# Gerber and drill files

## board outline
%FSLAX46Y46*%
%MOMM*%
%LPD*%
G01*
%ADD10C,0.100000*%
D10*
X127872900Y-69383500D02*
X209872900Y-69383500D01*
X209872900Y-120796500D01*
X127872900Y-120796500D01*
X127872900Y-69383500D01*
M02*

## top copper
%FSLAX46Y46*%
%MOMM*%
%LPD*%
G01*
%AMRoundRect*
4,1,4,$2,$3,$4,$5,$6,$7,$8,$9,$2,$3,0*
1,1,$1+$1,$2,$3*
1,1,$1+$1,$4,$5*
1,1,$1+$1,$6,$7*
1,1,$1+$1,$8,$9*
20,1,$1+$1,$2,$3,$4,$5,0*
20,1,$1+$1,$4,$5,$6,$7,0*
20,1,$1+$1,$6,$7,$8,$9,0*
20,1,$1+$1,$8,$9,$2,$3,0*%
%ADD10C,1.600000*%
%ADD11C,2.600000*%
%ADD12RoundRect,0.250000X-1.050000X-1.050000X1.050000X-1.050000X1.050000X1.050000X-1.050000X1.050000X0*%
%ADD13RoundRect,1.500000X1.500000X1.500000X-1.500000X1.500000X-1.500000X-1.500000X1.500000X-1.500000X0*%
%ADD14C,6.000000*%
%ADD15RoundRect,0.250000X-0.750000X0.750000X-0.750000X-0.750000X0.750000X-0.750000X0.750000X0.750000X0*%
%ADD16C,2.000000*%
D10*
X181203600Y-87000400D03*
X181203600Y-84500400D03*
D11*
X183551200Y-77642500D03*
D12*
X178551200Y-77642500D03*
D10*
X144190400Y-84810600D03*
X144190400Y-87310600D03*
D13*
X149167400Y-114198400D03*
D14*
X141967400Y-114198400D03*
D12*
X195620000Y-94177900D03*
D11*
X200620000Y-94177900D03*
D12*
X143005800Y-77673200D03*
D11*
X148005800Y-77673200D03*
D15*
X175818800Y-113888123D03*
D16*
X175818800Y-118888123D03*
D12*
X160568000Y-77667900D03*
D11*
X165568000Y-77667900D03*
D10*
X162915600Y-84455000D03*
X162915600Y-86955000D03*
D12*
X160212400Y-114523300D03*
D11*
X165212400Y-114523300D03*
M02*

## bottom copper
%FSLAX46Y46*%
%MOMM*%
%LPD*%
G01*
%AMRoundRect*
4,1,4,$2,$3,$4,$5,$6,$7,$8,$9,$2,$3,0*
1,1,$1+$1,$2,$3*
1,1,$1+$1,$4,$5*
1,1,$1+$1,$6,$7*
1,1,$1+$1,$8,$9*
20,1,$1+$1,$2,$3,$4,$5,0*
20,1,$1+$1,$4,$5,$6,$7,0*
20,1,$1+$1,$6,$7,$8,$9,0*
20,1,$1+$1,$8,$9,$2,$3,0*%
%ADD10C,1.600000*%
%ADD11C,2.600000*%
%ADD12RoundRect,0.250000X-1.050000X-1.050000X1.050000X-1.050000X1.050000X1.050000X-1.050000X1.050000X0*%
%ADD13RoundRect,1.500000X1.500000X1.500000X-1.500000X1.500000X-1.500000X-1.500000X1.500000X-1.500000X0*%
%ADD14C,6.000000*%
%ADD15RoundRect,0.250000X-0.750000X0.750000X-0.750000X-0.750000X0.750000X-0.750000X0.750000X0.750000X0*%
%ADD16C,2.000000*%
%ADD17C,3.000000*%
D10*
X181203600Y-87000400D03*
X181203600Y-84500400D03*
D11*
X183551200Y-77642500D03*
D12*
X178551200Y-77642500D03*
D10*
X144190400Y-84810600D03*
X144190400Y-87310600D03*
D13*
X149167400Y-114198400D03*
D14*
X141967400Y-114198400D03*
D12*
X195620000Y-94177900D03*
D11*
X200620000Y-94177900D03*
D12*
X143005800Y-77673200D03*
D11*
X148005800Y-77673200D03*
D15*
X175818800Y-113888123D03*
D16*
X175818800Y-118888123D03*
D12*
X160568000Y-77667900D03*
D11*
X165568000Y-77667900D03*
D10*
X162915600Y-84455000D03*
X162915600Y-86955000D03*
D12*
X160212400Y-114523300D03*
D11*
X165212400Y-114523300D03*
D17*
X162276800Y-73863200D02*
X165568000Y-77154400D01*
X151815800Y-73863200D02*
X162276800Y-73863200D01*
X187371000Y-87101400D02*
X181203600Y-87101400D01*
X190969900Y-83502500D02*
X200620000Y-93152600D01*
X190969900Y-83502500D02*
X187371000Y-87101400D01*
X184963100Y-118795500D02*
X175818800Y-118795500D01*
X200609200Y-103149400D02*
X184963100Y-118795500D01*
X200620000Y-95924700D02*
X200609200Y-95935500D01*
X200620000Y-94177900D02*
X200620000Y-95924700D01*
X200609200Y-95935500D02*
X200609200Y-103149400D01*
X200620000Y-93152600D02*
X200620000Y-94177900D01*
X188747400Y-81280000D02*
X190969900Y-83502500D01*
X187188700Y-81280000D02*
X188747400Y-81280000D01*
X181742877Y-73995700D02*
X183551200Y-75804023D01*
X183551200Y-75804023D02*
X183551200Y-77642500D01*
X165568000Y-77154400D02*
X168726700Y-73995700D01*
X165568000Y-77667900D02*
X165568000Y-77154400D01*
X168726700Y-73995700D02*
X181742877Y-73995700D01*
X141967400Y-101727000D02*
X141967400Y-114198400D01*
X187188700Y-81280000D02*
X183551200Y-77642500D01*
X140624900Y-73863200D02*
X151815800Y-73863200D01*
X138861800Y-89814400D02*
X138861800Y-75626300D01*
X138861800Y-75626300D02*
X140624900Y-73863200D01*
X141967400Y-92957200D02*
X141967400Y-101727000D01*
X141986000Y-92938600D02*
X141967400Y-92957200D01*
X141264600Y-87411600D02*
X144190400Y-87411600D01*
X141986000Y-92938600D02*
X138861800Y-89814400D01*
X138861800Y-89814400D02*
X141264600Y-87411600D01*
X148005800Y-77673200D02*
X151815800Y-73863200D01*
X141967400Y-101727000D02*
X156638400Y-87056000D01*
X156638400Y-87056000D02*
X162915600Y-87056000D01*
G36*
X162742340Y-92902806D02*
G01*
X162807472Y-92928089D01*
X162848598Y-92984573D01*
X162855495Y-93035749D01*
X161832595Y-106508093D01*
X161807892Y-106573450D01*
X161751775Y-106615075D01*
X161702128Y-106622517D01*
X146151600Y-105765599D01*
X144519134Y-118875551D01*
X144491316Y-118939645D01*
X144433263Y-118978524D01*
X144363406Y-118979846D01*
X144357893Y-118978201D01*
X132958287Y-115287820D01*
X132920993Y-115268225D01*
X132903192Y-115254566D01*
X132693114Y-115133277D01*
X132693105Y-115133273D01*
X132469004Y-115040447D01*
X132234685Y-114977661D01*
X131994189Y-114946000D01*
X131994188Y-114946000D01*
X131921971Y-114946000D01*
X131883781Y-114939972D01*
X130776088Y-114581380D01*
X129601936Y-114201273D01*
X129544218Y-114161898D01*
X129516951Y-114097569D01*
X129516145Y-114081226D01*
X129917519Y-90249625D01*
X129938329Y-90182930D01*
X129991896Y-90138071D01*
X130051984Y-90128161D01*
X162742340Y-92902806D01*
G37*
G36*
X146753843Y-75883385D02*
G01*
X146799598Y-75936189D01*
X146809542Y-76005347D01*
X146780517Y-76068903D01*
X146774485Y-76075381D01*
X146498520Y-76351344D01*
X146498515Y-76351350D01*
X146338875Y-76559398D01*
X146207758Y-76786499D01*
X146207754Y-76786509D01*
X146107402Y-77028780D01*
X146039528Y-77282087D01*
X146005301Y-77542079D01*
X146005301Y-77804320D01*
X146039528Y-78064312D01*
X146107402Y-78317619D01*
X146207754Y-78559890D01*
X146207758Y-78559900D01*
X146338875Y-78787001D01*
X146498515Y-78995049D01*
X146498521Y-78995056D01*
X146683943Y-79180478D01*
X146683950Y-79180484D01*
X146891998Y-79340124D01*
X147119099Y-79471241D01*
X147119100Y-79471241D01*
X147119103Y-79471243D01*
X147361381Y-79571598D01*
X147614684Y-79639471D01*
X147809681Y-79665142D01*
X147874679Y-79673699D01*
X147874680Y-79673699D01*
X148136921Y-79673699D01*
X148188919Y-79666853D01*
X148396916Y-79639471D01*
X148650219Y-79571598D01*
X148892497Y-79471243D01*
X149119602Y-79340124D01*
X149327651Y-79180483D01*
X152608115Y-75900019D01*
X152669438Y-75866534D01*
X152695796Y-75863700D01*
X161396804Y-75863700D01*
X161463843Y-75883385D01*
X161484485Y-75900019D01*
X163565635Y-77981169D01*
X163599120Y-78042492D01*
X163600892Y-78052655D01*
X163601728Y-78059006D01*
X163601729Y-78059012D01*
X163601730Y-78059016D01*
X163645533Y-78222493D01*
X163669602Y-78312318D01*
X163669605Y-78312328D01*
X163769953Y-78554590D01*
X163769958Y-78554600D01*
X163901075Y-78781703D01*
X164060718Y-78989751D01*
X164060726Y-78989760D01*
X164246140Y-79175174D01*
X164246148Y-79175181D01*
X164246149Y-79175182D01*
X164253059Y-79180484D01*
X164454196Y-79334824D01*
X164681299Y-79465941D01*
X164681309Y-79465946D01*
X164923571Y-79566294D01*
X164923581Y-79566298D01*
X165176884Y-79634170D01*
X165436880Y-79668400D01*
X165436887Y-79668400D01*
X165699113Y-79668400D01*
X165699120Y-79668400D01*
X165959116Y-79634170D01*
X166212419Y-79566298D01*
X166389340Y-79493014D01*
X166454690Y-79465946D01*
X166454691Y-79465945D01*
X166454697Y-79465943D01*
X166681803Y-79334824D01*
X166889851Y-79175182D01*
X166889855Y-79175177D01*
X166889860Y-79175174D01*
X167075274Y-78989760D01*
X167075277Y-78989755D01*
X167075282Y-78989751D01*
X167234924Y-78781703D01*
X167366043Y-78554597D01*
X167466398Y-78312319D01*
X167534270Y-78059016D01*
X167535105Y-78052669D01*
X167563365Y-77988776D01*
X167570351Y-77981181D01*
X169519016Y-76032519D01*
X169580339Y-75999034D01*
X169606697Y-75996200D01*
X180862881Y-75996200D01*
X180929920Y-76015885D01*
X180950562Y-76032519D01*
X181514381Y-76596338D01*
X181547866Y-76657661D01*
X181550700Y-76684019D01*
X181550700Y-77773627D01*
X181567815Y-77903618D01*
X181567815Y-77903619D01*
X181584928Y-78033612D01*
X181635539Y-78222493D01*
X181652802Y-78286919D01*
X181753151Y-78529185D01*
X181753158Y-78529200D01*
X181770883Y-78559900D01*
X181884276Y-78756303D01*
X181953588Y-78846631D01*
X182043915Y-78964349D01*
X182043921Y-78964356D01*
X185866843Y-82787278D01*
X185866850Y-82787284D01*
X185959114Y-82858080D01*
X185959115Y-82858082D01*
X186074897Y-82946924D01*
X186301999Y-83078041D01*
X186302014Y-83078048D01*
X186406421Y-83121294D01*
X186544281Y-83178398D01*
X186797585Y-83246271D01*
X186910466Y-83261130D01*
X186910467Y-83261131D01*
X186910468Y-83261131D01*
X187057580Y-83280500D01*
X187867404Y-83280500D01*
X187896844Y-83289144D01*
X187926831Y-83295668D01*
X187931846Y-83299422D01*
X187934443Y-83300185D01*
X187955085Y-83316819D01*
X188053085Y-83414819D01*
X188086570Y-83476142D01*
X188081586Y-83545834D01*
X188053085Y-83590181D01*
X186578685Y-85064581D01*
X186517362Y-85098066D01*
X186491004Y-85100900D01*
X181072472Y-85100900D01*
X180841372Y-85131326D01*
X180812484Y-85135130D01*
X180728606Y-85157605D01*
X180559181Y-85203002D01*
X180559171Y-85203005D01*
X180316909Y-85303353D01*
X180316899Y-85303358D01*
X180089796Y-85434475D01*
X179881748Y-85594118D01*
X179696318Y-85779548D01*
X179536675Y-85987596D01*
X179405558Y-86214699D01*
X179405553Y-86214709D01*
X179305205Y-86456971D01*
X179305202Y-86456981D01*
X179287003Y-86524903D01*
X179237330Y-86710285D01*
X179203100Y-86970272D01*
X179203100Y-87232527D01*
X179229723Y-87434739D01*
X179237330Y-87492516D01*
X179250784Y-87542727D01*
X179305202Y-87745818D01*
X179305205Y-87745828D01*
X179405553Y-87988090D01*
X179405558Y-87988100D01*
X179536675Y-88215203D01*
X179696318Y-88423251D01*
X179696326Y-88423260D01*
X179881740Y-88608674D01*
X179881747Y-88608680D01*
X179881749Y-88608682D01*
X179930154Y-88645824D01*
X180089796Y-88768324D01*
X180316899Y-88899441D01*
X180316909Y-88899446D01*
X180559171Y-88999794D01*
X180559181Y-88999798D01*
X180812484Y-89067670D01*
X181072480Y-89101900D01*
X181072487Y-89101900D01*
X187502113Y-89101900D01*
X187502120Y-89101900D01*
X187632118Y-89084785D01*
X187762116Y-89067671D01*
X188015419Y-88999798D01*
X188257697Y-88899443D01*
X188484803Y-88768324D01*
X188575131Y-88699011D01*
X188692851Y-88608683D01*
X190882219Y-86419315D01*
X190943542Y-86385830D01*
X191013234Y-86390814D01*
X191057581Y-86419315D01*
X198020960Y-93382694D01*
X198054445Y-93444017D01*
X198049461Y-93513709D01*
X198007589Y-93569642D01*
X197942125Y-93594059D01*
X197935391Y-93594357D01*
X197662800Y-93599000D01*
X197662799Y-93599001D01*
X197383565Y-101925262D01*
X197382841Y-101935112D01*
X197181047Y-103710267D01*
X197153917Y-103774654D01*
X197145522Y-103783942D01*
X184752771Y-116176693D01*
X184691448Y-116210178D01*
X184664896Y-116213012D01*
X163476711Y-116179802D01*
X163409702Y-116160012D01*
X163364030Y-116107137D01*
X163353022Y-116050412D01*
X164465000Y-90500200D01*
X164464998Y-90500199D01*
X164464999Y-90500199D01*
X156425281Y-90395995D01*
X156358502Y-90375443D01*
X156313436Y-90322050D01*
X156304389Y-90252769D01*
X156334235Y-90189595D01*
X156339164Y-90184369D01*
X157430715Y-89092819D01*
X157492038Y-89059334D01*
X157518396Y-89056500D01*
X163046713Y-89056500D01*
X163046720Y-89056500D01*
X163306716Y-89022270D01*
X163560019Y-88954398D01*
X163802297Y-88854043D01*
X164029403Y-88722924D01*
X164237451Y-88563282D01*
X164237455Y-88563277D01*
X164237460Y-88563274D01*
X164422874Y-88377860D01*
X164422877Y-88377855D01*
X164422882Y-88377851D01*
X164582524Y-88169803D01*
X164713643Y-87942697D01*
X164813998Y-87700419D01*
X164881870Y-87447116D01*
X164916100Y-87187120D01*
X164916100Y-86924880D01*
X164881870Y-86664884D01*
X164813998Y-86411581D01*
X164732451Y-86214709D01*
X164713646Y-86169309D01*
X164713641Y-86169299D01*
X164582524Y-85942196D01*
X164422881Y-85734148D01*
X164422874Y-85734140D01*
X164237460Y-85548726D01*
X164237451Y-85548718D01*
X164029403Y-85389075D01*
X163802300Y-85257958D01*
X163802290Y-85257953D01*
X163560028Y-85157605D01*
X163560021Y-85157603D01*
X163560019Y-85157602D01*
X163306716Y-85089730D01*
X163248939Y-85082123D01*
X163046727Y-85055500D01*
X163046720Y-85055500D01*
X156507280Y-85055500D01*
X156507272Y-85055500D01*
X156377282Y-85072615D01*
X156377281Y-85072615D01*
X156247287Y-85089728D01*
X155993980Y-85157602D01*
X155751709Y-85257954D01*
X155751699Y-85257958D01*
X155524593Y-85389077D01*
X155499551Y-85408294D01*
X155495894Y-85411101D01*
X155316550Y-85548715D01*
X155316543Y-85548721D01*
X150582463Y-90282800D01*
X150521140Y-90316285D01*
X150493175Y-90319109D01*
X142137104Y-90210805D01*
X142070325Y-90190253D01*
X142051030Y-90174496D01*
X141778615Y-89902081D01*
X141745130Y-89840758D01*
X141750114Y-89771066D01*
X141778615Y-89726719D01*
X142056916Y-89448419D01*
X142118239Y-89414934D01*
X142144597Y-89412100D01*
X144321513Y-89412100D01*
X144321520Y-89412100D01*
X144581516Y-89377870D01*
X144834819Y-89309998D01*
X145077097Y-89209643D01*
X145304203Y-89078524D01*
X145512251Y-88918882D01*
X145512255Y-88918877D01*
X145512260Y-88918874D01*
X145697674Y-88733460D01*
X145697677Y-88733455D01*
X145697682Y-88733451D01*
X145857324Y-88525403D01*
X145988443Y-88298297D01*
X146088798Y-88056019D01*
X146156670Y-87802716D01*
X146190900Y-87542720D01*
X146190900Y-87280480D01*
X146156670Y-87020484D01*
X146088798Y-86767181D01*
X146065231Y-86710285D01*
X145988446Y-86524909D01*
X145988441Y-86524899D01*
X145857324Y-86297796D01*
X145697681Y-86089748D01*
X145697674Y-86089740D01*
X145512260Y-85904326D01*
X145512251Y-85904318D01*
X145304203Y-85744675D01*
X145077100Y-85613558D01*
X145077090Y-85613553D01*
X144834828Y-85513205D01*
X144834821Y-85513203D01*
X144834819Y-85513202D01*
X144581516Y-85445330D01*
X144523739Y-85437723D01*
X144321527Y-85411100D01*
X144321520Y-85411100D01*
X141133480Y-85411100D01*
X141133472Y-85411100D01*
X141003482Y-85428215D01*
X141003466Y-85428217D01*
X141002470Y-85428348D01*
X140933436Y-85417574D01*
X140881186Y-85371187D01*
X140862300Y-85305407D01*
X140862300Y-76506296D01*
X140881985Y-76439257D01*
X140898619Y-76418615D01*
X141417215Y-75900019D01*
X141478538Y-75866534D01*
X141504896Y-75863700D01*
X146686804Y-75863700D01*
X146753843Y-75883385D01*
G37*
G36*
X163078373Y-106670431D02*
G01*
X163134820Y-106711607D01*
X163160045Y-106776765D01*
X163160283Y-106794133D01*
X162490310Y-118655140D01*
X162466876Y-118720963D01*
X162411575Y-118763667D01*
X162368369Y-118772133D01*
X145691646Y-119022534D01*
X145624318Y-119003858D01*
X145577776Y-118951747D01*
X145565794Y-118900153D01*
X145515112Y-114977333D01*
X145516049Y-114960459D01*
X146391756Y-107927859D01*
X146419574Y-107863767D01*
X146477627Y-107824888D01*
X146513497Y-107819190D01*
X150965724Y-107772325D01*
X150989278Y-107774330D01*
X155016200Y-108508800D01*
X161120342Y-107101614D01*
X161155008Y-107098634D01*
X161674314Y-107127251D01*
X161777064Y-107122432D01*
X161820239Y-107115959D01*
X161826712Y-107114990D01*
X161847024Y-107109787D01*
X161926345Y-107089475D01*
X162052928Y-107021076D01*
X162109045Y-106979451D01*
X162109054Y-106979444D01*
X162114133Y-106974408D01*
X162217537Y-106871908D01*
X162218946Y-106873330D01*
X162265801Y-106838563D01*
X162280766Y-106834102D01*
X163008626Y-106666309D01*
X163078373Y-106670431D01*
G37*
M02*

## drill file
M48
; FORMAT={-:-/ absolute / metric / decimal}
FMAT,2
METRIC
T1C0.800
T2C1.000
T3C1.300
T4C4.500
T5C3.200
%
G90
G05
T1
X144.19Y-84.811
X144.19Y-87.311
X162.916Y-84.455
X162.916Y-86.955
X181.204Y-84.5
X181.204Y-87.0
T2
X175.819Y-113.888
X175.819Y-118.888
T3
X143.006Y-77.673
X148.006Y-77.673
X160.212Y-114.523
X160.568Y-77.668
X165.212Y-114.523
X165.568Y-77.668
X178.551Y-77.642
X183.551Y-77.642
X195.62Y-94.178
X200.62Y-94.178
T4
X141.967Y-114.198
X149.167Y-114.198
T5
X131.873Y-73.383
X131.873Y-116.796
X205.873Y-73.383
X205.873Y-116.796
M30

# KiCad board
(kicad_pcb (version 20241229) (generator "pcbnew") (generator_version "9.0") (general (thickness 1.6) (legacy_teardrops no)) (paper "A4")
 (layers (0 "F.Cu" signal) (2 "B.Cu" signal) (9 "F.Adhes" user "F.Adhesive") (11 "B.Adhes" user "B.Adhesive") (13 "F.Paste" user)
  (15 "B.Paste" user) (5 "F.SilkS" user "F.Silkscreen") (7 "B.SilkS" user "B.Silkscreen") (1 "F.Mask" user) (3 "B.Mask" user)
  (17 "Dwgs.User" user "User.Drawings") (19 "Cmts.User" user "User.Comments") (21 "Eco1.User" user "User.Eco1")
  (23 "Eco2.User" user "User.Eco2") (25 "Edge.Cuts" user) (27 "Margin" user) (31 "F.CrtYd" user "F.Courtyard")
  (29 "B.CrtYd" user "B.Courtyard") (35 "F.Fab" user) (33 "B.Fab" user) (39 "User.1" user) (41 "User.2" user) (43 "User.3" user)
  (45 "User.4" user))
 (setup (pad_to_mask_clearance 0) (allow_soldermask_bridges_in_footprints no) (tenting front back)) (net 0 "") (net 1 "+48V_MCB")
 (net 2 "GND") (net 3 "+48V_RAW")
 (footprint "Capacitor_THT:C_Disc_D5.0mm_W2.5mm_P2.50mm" (layer "F.Cu") (at 144.1904 84.8106 -90)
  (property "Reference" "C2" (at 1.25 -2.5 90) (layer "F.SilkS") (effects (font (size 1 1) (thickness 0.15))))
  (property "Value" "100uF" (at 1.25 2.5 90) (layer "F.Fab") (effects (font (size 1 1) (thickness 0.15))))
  (pad "1" thru_hole circle (at 0 0 270) (size 1.6 1.6) (drill 0.8) (layers "*.Cu" "*.Mask") (remove_unused_layers no) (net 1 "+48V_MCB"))
  (pad "2" thru_hole circle (at 2.5 0 270) (size 1.6 1.6) (drill 0.8) (layers "*.Cu" "*.Mask") (remove_unused_layers no) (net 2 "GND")))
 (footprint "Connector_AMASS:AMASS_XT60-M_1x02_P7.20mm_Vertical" (layer "F.Cu") (at 149.1674 114.1984 180)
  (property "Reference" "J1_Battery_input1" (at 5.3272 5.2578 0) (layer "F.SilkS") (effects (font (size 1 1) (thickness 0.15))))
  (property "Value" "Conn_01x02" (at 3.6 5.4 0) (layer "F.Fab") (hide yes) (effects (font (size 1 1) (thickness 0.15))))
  (pad "1" thru_hole roundrect (at 0 0 180) (size 6 6) (drill 4.5) (layers "*.Cu" "*.Mask") (remove_unused_layers no)
   (roundrect_rratio 0.25) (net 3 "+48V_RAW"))
  (pad "2" thru_hole circle (at 7.2 0 180) (size 6 6) (drill 4.5) (layers "*.Cu" "*.Mask") (remove_unused_layers no) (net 2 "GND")))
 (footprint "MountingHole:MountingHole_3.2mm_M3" (layer "F.Cu") (at 131.8729 116.7965)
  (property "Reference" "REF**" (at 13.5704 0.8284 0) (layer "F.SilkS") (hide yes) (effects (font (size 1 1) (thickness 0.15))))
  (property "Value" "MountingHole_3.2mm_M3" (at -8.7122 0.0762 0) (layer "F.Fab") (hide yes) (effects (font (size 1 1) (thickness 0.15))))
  (pad "" np_thru_hole circle (at 0 0) (size 3.2 3.2) (drill 3.2) (layers "*.Cu" "*.Mask")))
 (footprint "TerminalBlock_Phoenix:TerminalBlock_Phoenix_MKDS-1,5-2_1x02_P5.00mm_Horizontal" (layer "F.Cu") (at 160.2124 114.5233)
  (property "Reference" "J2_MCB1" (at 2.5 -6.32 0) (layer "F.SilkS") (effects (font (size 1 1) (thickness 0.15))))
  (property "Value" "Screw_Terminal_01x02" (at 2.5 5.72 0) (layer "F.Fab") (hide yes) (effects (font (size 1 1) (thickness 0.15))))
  (pad "1" thru_hole roundrect (at 0 0) (size 2.6 2.6) (drill 1.3) (layers "*.Cu" "*.Mask") (remove_unused_layers no)
   (roundrect_rratio 0.096154) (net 3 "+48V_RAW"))
  (pad "2" thru_hole circle (at 5 0) (size 2.6 2.6) (drill 1.3) (layers "*.Cu" "*.Mask") (remove_unused_layers no) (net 1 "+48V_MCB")))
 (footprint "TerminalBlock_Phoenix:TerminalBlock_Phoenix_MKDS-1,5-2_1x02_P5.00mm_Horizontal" (layer "F.Cu") (at 195.62 94.1779)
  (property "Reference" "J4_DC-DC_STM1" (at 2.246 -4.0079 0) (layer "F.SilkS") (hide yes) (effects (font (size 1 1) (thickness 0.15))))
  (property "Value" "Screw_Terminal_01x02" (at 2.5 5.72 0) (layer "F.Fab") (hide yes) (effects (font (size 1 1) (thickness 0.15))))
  (pad "1" thru_hole roundrect (at 0 0) (size 2.6 2.6) (drill 1.3) (layers "*.Cu" "*.Mask") (remove_unused_layers no)
   (roundrect_rratio 0.096154) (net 1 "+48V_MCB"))
  (pad "2" thru_hole circle (at 5 0) (size 2.6 2.6) (drill 1.3) (layers "*.Cu" "*.Mask") (remove_unused_layers no) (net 2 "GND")))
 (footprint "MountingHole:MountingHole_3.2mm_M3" (layer "F.Cu") (at 131.8729 73.3835)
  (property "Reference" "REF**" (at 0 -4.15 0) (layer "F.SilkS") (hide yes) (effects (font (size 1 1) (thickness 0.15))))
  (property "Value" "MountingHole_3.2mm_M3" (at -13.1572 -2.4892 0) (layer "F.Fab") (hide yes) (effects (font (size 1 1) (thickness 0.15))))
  (pad "" np_thru_hole circle (at 0 0) (size 3.2 3.2) (drill 3.2) (layers "*.Cu" "*.Mask")))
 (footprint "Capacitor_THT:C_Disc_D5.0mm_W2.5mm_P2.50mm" (layer "F.Cu") (at 181.2036 84.5004 -90)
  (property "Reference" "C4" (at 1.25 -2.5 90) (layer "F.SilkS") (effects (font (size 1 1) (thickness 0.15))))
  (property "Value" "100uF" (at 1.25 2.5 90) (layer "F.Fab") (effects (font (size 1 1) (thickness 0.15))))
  (pad "1" thru_hole circle (at 0 0 270) (size 1.6 1.6) (drill 0.8) (layers "*.Cu" "*.Mask") (remove_unused_layers no) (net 1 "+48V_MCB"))
  (pad "2" thru_hole circle (at 2.5 0 270) (size 1.6 1.6) (drill 0.8) (layers "*.Cu" "*.Mask") (remove_unused_layers no) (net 2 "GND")))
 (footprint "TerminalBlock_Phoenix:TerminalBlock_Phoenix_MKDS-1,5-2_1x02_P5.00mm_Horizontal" (layer "F.Cu") (at 143.0058 77.6732)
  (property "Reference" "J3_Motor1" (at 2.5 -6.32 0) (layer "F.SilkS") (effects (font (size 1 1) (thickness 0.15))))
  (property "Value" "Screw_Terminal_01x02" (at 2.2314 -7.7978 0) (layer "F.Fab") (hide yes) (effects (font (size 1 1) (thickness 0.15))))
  (pad "1" thru_hole roundrect (at 0 0) (size 2.6 2.6) (drill 1.3) (layers "*.Cu" "*.Mask") (remove_unused_layers no)
   (roundrect_rratio 0.096154) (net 1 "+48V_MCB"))
  (pad "2" thru_hole circle (at 5 0) (size 2.6 2.6) (drill 1.3) (layers "*.Cu" "*.Mask") (remove_unused_layers no) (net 2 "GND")))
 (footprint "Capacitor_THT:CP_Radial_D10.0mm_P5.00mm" (layer "F.Cu") (at 175.8188 113.888123 -90)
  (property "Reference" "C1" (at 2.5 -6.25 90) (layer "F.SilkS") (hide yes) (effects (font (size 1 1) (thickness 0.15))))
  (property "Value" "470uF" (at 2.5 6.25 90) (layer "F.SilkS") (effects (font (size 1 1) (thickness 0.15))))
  (pad "1" thru_hole roundrect (at 0 0 270) (size 2 2) (drill 1) (layers "*.Cu" "*.Mask") (remove_unused_layers no) (roundrect_rratio 0.125)
   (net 1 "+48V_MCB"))
  (pad "2" thru_hole circle (at 5 0 270) (size 2 2) (drill 1) (layers "*.Cu" "*.Mask") (remove_unused_layers no) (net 2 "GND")))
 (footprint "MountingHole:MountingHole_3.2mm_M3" (layer "F.Cu") (at 205.8729 116.7965)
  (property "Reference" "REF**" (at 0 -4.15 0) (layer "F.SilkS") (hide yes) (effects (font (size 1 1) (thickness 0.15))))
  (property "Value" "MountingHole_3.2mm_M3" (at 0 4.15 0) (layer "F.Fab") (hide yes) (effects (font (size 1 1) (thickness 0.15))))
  (pad "" np_thru_hole circle (at 0 0) (size 3.2 3.2) (drill 3.2) (layers "*.Cu" "*.Mask")))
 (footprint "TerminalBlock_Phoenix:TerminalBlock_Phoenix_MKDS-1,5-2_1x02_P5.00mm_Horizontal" (layer "F.Cu") (at 160.568 77.6679)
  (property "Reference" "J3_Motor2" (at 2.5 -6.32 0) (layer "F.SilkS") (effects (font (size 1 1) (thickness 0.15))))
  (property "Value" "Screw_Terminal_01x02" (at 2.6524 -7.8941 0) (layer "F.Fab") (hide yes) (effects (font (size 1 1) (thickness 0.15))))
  (pad "1" thru_hole roundrect (at 0 0) (size 2.6 2.6) (drill 1.3) (layers "*.Cu" "*.Mask") (remove_unused_layers no)
   (roundrect_rratio 0.096154) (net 1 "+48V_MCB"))
  (pad "2" thru_hole circle (at 5 0) (size 2.6 2.6) (drill 1.3) (layers "*.Cu" "*.Mask") (remove_unused_layers no) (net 2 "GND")))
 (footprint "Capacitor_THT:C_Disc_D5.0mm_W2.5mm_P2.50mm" (layer "F.Cu") (at 162.9156 84.455 -90)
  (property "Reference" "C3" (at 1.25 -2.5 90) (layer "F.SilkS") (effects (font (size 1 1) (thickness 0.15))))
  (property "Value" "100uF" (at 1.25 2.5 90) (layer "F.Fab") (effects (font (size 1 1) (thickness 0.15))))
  (pad "1" thru_hole circle (at 0 0 270) (size 1.6 1.6) (drill 0.8) (layers "*.Cu" "*.Mask") (remove_unused_layers no) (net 1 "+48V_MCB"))
  (pad "2" thru_hole circle (at 2.5 0 270) (size 1.6 1.6) (drill 0.8) (layers "*.Cu" "*.Mask") (remove_unused_layers no) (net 2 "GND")))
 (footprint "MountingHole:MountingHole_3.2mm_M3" (layer "F.Cu") (at 205.8729 73.3835)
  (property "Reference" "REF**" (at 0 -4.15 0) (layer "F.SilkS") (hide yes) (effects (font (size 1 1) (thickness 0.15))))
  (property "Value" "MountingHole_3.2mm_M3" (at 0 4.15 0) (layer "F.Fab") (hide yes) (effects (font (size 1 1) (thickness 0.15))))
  (pad "" np_thru_hole circle (at 0 0) (size 3.2 3.2) (drill 3.2) (layers "*.Cu" "*.Mask")))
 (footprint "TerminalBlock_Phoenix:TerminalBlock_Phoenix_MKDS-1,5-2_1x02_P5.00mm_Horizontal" (layer "F.Cu") (at 178.5512 77.6425)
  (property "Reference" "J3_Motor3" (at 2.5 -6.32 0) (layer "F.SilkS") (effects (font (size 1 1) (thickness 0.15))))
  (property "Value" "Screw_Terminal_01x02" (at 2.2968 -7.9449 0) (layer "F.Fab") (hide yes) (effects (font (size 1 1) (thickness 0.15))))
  (pad "1" thru_hole roundrect (at 0 0) (size 2.6 2.6) (drill 1.3) (layers "*.Cu" "*.Mask") (remove_unused_layers no)
   (roundrect_rratio 0.096154) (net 1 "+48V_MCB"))
  (pad "2" thru_hole circle (at 5 0) (size 2.6 2.6) (drill 1.3) (layers "*.Cu" "*.Mask") (remove_unused_layers no) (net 2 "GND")))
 (gr_rect (start 127.8729 69.3835) (end 209.8729 120.7965) (stroke (width 0.1) (type solid)) (fill no) (layer "Edge.Cuts"))
 (segment (start 156.6384 87.056) (end 162.9156 87.056) (width 3) (layer "B.Cu") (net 2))
 (segment (start 148.0058 77.6732) (end 151.8158 73.8632) (width 3) (layer "B.Cu") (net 2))
 (segment (start 141.986 92.9386) (end 138.8618 89.8144) (width 3) (layer "B.Cu") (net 2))
 (segment (start 141.2646 87.4116) (end 144.1904 87.4116) (width 3) (layer "B.Cu") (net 2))
 (segment (start 183.5512 75.804023) (end 183.5512 77.6425) (width 3) (layer "B.Cu") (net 2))
 (segment (start 141.9674 101.727) (end 156.6384 87.056) (width 3) (layer "B.Cu") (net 2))
 (segment (start 200.62 95.9247) (end 200.6092 95.9355) (width 3) (layer "B.Cu") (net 2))
 (segment (start 200.6092 95.9355) (end 200.6092 103.1494) (width 3) (layer "B.Cu") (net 2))
 (segment (start 138.8618 89.8144) (end 141.2646 87.4116) (width 3) (layer "B.Cu") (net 2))
 (segment (start 188.7474 81.28) (end 190.9699 83.5025) (width 3) (layer "B.Cu") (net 2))
 (segment (start 187.1887 81.28) (end 183.5512 77.6425) (width 3) (layer "B.Cu") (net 2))
 (segment (start 138.8618 89.8144) (end 138.8618 75.6263) (width 3) (layer "B.Cu") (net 2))
 (segment (start 187.1887 81.28) (end 188.7474 81.28) (width 3) (layer "B.Cu") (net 2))
 (segment (start 141.986 92.9386) (end 141.9674 92.9572) (width 3) (layer "B.Cu") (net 2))
 (segment (start 162.2768 73.8632) (end 165.568 77.1544) (width 3) (layer "B.Cu") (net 2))
 (segment (start 138.8618 75.6263) (end 140.6249 73.8632) (width 3) (layer "B.Cu") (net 2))
 (segment (start 200.62 93.1526) (end 200.62 94.1779) (width 3) (layer "B.Cu") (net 2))
 (segment (start 141.9674 101.727) (end 141.9674 114.1984) (width 3) (layer "B.Cu") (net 2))
 (segment (start 140.6249 73.8632) (end 151.8158 73.8632) (width 3) (layer "B.Cu") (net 2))
 (segment (start 165.568 77.6679) (end 165.568 77.1544) (width 3) (layer "B.Cu") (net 2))
 (segment (start 187.371 87.1014) (end 181.2036 87.1014) (width 3) (layer "B.Cu") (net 2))
 (segment (start 184.9631 118.7955) (end 175.8188 118.7955) (width 3) (layer "B.Cu") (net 2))
 (segment (start 200.62 94.1779) (end 200.62 95.9247) (width 3) (layer "B.Cu") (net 2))
 (segment (start 141.9674 92.9572) (end 141.9674 101.727) (width 3) (layer "B.Cu") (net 2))
 (segment (start 190.9699 83.5025) (end 200.62 93.1526) (width 3) (layer "B.Cu") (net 2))
 (segment (start 165.568 77.1544) (end 168.7267 73.9957) (width 3) (layer "B.Cu") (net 2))
 (segment (start 181.742877 73.9957) (end 183.5512 75.804023) (width 3) (layer "B.Cu") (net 2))
 (segment (start 151.8158 73.8632) (end 162.2768 73.8632) (width 3) (layer "B.Cu") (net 2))
 (segment (start 168.7267 73.9957) (end 181.742877 73.9957) (width 3) (layer "B.Cu") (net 2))
 (segment (start 200.6092 103.1494) (end 184.9631 118.7955) (width 3) (layer "B.Cu") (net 2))
 (segment (start 190.9699 83.5025) (end 187.371 87.1014) (width 3) (layer "B.Cu") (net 2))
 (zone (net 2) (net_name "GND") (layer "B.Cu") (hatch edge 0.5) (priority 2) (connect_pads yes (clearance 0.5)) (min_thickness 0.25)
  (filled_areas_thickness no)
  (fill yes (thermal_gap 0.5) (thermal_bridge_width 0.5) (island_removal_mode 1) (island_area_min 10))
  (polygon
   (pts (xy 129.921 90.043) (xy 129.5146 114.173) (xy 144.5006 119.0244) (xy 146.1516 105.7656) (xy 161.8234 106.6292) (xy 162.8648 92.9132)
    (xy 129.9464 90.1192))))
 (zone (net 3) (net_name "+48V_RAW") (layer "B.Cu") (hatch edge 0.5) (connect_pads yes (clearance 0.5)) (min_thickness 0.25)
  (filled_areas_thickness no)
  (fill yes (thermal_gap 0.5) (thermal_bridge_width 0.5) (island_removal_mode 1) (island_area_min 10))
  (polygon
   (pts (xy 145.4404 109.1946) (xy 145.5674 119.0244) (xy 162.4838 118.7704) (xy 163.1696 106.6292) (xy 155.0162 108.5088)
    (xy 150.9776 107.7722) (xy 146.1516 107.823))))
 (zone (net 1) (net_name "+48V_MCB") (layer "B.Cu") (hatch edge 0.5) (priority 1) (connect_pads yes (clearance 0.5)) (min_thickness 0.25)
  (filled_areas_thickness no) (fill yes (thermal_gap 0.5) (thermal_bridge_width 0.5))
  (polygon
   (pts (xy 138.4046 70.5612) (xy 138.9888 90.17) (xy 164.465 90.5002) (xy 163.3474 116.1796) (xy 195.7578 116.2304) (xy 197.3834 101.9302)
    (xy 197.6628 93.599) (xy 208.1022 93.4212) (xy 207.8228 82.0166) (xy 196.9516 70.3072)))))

